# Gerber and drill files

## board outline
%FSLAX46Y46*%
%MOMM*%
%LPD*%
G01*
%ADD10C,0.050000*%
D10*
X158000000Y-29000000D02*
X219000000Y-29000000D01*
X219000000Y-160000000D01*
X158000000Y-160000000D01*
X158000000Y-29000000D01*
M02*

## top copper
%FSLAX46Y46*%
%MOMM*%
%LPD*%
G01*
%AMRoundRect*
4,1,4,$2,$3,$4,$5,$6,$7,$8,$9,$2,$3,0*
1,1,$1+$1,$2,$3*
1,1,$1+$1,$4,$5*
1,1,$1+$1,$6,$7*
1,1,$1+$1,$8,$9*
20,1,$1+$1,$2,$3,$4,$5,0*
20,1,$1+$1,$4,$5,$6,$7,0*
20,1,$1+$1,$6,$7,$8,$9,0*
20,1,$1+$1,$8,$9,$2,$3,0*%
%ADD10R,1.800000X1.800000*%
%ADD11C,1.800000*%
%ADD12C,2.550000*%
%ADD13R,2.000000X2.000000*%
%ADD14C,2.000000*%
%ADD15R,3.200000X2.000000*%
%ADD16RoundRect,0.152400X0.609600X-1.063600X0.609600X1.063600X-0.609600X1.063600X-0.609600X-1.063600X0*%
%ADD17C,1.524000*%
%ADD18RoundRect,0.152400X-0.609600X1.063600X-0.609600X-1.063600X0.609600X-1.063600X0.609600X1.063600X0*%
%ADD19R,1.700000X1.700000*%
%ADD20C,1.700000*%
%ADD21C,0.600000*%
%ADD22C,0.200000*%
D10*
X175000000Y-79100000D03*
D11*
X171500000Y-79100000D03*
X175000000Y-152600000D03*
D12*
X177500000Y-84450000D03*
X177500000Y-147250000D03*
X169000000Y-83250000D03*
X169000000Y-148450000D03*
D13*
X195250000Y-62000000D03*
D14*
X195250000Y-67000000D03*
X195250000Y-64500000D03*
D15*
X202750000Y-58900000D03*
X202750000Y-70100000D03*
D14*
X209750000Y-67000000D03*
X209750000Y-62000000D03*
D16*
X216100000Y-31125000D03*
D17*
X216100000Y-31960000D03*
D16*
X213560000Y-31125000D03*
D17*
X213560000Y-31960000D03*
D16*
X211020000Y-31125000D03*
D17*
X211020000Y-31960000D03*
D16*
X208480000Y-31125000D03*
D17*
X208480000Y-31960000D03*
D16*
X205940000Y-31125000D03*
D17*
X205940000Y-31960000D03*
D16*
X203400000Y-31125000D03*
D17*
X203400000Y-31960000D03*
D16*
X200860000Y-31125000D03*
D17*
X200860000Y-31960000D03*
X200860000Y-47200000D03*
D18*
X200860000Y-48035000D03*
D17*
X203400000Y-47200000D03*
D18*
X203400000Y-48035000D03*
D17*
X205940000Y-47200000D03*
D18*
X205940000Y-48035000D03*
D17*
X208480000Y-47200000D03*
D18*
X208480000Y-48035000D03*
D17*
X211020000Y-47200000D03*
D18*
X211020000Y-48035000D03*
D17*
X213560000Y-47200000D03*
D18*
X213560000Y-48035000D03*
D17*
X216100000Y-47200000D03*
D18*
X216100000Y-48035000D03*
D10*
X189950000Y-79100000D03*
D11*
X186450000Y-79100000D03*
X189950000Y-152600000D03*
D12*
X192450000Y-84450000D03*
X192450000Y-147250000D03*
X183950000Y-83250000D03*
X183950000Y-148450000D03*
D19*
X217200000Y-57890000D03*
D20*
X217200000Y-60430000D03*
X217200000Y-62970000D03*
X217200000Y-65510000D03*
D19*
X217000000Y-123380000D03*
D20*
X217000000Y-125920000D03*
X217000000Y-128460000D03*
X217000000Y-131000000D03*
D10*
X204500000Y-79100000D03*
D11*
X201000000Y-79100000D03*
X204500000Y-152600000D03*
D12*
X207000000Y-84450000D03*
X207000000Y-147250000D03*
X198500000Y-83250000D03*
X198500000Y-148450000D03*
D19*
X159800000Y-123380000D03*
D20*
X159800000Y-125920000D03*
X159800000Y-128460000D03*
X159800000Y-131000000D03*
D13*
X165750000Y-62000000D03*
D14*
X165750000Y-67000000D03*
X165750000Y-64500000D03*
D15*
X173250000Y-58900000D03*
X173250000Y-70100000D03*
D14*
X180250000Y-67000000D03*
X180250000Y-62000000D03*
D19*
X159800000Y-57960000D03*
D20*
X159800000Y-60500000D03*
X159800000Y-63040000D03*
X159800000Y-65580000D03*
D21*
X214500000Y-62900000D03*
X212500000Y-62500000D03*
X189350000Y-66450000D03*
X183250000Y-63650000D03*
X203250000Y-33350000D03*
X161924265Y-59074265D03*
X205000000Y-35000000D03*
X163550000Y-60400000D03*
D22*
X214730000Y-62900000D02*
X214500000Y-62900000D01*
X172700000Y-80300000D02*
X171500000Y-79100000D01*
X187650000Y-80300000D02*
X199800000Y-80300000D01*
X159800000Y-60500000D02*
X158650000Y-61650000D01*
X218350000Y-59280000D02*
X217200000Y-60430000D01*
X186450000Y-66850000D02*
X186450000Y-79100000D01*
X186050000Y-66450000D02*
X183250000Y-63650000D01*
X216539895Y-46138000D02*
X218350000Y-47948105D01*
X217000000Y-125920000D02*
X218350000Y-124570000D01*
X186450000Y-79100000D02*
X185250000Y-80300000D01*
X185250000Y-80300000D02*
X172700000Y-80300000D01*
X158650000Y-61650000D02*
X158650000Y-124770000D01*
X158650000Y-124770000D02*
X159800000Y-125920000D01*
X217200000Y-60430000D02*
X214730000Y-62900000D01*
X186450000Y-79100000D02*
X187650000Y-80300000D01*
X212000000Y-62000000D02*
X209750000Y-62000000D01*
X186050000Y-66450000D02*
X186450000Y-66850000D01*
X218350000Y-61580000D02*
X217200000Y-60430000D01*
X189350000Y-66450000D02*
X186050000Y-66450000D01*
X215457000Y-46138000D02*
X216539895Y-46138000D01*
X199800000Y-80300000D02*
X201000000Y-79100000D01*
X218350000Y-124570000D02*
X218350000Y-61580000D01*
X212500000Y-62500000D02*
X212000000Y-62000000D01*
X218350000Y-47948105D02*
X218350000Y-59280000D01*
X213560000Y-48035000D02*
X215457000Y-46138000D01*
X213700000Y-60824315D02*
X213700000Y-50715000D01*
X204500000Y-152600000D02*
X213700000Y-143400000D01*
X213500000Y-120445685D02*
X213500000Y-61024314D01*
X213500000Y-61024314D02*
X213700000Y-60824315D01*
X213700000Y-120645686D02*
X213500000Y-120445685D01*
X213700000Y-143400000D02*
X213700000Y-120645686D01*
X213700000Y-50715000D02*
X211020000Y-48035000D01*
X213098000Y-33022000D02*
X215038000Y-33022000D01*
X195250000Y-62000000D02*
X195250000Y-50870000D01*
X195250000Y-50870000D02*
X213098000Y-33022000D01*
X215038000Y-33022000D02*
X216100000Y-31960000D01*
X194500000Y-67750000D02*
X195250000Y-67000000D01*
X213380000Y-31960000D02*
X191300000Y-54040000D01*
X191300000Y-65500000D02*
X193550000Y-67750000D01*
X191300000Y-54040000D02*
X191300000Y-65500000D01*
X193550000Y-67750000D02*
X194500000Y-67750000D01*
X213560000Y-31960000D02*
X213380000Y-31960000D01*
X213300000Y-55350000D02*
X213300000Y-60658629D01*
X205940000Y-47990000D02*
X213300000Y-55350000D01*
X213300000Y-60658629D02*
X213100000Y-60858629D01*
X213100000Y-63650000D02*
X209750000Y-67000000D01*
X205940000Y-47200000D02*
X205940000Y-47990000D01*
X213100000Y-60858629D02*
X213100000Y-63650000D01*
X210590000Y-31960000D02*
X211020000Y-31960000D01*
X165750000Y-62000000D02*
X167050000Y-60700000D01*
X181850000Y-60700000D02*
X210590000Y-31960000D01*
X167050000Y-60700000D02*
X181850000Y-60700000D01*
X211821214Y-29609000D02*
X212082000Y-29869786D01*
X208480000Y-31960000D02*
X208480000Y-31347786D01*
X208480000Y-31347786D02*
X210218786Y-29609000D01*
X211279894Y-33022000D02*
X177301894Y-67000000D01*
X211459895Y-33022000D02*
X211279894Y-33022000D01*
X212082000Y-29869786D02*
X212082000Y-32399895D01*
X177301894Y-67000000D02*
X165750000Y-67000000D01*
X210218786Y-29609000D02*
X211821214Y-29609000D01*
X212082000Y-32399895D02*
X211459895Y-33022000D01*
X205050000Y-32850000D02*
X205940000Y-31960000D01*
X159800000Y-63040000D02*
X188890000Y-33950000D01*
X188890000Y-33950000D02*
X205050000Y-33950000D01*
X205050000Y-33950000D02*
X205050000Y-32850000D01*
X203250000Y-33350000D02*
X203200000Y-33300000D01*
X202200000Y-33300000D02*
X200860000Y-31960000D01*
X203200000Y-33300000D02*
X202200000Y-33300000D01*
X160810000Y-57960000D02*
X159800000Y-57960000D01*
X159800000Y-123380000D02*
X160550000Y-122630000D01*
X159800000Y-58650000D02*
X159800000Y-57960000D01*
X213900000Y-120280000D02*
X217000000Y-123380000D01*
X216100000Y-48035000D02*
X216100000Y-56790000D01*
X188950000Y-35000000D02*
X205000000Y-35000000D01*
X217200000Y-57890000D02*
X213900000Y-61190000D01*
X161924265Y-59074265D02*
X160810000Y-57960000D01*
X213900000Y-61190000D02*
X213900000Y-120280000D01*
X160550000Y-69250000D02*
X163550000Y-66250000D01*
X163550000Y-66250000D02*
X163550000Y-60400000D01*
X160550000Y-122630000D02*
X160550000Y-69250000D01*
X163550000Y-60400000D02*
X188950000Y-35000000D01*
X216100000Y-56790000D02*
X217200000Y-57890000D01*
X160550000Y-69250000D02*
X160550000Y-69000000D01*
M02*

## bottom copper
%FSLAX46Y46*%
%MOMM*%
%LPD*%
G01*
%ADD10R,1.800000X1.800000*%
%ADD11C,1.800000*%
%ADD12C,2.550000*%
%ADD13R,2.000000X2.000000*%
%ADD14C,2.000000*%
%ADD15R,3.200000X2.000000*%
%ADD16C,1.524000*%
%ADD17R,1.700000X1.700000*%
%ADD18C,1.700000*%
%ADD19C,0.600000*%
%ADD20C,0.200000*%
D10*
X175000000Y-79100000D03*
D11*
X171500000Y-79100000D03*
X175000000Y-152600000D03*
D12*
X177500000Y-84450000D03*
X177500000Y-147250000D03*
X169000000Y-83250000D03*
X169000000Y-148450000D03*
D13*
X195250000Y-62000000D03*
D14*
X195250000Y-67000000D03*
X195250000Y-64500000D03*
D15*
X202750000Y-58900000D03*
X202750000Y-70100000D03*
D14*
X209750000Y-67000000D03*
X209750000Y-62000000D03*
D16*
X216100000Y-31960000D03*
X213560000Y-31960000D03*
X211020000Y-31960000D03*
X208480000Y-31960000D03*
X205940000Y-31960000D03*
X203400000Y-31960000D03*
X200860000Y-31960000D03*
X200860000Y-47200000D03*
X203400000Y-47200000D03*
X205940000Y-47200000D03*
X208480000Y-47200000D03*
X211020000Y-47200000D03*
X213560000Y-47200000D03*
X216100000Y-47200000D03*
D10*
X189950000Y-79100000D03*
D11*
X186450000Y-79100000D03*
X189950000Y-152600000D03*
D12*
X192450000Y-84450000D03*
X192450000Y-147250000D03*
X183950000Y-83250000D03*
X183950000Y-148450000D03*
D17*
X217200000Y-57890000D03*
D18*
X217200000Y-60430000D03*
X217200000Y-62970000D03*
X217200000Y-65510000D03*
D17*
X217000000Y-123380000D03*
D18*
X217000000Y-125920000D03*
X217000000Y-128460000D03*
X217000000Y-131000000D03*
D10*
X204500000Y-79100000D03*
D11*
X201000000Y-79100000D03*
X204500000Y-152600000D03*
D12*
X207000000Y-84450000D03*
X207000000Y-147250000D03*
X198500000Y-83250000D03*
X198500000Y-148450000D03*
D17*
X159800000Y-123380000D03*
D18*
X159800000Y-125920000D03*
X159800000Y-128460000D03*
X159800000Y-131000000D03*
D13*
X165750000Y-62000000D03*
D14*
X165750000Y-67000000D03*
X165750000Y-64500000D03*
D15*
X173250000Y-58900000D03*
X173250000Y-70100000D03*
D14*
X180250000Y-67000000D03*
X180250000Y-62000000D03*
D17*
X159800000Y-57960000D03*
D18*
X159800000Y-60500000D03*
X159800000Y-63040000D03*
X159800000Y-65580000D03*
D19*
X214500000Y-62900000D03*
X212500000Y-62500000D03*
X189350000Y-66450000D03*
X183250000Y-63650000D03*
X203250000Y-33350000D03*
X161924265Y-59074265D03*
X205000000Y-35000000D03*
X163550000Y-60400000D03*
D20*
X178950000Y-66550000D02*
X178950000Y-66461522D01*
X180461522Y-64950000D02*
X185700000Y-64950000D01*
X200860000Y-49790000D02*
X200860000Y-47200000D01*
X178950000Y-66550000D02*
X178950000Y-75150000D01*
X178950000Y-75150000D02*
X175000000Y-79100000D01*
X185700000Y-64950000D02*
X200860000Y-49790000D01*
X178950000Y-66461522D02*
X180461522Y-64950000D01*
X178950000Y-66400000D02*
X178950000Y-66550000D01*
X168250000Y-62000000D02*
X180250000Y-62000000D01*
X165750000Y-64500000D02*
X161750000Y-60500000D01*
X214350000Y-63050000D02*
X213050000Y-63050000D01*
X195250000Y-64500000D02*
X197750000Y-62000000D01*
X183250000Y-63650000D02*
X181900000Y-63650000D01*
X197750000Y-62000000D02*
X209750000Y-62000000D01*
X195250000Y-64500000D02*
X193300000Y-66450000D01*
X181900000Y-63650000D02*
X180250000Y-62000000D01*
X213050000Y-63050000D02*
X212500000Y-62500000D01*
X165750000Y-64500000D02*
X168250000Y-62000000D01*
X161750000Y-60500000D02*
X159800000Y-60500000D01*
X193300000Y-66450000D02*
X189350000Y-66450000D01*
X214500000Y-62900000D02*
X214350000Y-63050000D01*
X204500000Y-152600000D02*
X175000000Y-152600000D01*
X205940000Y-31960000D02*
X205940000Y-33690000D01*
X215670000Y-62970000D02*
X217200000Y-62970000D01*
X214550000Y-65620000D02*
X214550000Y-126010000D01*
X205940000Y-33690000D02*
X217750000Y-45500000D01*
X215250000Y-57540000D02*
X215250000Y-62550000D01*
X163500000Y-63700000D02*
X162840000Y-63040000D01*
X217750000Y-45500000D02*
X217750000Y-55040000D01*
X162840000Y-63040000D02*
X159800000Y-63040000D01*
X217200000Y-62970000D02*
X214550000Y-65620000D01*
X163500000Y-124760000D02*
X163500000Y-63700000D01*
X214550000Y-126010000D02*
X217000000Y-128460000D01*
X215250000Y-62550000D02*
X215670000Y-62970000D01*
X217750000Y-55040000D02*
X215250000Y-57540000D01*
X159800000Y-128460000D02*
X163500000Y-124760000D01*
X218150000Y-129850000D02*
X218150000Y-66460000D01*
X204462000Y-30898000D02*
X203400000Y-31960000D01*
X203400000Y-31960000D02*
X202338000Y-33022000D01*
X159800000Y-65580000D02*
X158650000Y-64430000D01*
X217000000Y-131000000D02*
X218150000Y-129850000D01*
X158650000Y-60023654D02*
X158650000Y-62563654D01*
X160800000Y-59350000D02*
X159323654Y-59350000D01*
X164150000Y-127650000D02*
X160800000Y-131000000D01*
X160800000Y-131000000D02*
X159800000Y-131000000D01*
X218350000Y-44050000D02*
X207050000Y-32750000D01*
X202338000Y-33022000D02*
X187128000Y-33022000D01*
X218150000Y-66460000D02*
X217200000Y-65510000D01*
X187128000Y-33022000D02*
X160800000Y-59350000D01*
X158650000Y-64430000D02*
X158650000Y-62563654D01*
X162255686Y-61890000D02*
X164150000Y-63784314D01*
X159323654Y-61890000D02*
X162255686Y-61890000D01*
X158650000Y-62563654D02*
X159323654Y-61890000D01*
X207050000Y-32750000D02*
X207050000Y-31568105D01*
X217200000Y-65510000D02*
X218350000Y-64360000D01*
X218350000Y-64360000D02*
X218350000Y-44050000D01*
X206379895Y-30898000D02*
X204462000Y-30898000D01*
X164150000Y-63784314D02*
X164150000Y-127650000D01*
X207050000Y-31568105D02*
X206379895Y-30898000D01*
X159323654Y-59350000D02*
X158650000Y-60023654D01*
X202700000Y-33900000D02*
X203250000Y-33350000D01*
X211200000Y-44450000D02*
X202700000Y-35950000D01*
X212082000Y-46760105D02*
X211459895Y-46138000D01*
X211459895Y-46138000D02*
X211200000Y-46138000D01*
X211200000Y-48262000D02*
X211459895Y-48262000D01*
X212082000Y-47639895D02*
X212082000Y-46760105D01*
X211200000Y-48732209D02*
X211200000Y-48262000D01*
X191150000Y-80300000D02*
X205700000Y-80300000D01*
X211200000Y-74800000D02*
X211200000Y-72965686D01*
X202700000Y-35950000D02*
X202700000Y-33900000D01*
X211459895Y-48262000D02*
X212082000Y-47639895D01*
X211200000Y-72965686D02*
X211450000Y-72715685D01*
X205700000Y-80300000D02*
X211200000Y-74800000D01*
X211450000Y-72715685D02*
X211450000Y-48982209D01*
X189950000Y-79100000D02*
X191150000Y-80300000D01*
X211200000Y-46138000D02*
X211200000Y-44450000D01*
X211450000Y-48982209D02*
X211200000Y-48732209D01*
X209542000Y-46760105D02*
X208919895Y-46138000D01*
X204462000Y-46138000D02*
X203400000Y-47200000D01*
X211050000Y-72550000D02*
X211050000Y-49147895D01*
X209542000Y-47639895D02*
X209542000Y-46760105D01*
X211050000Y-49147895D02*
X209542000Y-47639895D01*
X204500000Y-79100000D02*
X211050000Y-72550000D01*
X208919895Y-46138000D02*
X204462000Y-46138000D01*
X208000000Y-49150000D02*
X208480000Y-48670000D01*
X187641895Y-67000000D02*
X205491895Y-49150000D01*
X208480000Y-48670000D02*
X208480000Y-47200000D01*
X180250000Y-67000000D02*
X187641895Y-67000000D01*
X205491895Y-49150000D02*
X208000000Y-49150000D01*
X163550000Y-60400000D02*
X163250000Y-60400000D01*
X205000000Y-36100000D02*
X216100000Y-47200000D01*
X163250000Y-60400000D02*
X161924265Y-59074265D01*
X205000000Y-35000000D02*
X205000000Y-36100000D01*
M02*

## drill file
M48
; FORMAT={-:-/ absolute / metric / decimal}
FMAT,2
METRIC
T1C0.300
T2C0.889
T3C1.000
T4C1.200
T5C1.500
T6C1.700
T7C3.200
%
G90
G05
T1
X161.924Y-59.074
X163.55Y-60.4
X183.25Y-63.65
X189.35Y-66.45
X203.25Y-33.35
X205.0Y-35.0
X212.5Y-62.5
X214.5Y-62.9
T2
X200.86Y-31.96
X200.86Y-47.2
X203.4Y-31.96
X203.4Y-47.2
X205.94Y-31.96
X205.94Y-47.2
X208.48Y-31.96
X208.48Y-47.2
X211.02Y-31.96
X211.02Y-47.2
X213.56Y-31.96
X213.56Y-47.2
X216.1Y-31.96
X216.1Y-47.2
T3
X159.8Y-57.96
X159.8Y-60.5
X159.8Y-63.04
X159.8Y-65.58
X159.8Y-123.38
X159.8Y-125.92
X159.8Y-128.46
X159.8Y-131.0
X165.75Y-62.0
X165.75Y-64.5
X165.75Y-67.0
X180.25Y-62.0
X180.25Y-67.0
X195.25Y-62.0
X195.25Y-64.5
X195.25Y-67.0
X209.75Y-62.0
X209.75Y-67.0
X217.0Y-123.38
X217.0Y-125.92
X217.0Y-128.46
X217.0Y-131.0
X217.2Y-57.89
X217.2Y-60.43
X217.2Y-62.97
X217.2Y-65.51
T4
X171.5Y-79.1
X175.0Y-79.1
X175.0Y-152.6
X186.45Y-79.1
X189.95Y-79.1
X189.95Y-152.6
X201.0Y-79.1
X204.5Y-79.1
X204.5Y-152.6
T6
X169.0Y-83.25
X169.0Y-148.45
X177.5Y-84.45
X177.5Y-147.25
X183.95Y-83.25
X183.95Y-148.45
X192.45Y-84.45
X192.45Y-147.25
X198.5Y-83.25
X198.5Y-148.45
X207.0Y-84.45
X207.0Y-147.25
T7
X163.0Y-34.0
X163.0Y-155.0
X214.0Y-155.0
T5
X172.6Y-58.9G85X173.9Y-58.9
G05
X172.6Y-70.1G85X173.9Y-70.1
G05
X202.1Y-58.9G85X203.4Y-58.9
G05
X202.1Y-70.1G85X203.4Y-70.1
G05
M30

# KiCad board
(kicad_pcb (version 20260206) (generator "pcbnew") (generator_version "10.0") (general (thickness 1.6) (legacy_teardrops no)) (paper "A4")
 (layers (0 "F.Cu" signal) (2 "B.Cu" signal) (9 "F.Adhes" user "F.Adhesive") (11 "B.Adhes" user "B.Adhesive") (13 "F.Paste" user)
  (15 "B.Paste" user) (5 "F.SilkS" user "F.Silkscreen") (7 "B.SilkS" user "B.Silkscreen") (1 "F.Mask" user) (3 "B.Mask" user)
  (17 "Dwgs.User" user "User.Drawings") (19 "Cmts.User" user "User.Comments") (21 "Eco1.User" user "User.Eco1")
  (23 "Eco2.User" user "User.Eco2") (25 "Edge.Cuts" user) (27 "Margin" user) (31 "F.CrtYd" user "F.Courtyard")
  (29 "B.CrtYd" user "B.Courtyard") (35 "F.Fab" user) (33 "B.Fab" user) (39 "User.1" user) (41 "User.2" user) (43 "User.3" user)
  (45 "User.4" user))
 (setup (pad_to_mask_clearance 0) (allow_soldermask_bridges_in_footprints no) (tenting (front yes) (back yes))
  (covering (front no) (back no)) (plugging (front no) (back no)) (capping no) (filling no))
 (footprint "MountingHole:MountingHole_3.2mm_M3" (layer "F.Cu") (at 163 34)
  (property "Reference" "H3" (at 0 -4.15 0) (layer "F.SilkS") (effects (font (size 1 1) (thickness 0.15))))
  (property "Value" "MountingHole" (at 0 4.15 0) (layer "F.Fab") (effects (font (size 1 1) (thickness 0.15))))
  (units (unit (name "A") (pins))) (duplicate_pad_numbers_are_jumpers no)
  (pad "" np_thru_hole circle (at 0 0) (size 3.2 3.2) (drill 3.2) (layers "*.Cu" "*.Mask")))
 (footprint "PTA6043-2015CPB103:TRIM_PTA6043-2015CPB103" (layer "F.Cu") (at 173.25 115.85 -90)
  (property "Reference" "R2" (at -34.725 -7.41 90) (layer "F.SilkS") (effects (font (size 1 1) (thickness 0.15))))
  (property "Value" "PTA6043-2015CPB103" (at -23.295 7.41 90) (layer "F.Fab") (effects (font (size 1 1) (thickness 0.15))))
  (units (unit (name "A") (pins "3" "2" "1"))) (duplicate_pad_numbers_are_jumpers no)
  (pad "1" thru_hole rect (at -36.75 -1.75 270) (size 1.8 1.8) (drill 1.2) (layers "*.Cu" "*.Mask") (remove_unused_layers no) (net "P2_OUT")
   (solder_mask_margin 0.102))
  (pad "2" thru_hole circle (at -36.75 1.75 270) (size 1.8 1.8) (drill 1.2) (layers "*.Cu" "*.Mask") (remove_unused_layers no) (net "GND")
   (solder_mask_margin 0.102))
  (pad "3" thru_hole circle (at 36.75 -1.75 270) (size 1.8 1.8) (drill 1.2) (layers "*.Cu" "*.Mask") (remove_unused_layers no) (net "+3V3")
   (solder_mask_margin 0.102))
  (pad "SH1" thru_hole circle (at -31.4 -4.25 270) (size 2.55 2.55) (drill 1.7) (layers "*.Cu" "*.Mask") (remove_unused_layers no)
   (solder_mask_margin 0.102))
  (pad "SH2" thru_hole circle (at 31.4 -4.25 270) (size 2.55 2.55) (drill 1.7) (layers "*.Cu" "*.Mask") (remove_unused_layers no)
   (solder_mask_margin 0.102))
  (pad "SH3" thru_hole circle (at -32.6 4.25 270) (size 2.55 2.55) (drill 1.7) (layers "*.Cu" "*.Mask") (remove_unused_layers no)
   (solder_mask_margin 0.102))
  (pad "SH4" thru_hole circle (at 32.6 4.25 270) (size 2.55 2.55) (drill 1.7) (layers "*.Cu" "*.Mask") (remove_unused_layers no)
   (solder_mask_margin 0.102)))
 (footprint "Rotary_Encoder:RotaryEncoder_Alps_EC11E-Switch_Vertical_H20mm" (layer "F.Cu") (at 195.25 62)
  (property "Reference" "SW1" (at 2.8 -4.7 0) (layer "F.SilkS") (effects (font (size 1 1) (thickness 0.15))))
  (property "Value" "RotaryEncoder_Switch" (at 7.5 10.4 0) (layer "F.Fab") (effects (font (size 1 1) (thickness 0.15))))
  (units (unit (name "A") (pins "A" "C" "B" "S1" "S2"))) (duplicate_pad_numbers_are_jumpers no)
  (pad "A" thru_hole rect (at 0 0) (size 2 2) (drill 1) (layers "*.Cu" "*.Mask") (remove_unused_layers no) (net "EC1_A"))
  (pad "B" thru_hole circle (at 0 5) (size 2 2) (drill 1) (layers "*.Cu" "*.Mask") (remove_unused_layers no) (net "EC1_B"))
  (pad "C" thru_hole circle (at 0 2.5) (size 2 2) (drill 1) (layers "*.Cu" "*.Mask") (remove_unused_layers no) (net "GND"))
  (pad "MP" thru_hole rect (at 7.5 -3.1) (size 3.2 2) (drill oval 2.8 1.5) (layers "*.Cu" "*.Mask") (remove_unused_layers no))
  (pad "MP" thru_hole rect (at 7.5 8.1) (size 3.2 2) (drill oval 2.8 1.5) (layers "*.Cu" "*.Mask") (remove_unused_layers no))
  (pad "S1" thru_hole circle (at 14.5 5) (size 2 2) (drill 1) (layers "*.Cu" "*.Mask") (remove_unused_layers no) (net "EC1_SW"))
  (pad "S2" thru_hole circle (at 14.5 0) (size 2 2) (drill 1) (layers "*.Cu" "*.Mask") (remove_unused_layers no) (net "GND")))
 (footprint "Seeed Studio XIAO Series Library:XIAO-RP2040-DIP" (layer "F.Cu") (at 208.48 39.58)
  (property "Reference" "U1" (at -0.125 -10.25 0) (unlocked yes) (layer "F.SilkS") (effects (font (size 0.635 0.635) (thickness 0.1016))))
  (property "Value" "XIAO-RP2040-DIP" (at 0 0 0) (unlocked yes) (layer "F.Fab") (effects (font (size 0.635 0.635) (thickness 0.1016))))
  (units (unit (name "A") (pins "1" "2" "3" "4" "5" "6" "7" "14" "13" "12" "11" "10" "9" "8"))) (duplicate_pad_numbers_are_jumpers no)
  (pad "1" smd roundrect (at 7.62 -8.455 90) (size 2.432 1.524) (layers "F.Cu" "F.Mask") (roundrect_rratio 0.1) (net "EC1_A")
   (thermal_bridge_angle 45))
  (pad "1" thru_hole circle (at 7.62 -7.62 90) (size 1.524 1.524) (drill 0.889) (layers "*.Cu" "*.Mask") (remove_unused_layers no)
   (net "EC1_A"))
  (pad "2" smd roundrect (at 5.08 -8.455 90) (size 2.432 1.524) (layers "F.Cu" "F.Mask") (roundrect_rratio 0.1) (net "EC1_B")
   (thermal_bridge_angle 45))
  (pad "2" thru_hole circle (at 5.08 -7.62 90) (size 1.524 1.524) (drill 0.889) (layers "*.Cu" "*.Mask") (remove_unused_layers no)
   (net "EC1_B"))
  (pad "3" smd roundrect (at 2.54 -8.455 90) (size 2.432 1.524) (layers "F.Cu" "F.Mask") (roundrect_rratio 0.1) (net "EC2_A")
   (thermal_bridge_angle 45))
  (pad "3" thru_hole circle (at 2.54 -7.62 90) (size 1.524 1.524) (drill 0.889) (layers "*.Cu" "*.Mask") (remove_unused_layers no)
   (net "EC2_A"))
  (pad "4" smd roundrect (at 0 -8.455 90) (size 2.432 1.524) (layers "F.Cu" "F.Mask") (roundrect_rratio 0.1) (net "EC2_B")
   (thermal_bridge_angle 45))
  (pad "4" thru_hole circle (at 0 -7.62 90) (size 1.524 1.524) (drill 0.889) (layers "*.Cu" "*.Mask") (remove_unused_layers no)
   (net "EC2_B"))
  (pad "5" smd roundrect (at -2.54 -8.455 90) (size 2.432 1.524) (layers "F.Cu" "F.Mask") (roundrect_rratio 0.1) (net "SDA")
   (thermal_bridge_angle 45))
  (pad "5" thru_hole circle (at -2.54 -7.62 90) (size 1.524 1.524) (drill 0.889) (layers "*.Cu" "*.Mask") (remove_unused_layers no)
   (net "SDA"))
  (pad "6" smd roundrect (at -5.08 -8.455 90) (size 2.432 1.524) (layers "F.Cu" "F.Mask") (roundrect_rratio 0.1) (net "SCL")
   (thermal_bridge_angle 45))
  (pad "6" thru_hole circle (at -5.08 -7.62 90) (size 1.524 1.524) (drill 0.889) (layers "*.Cu" "*.Mask") (remove_unused_layers no)
   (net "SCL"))
  (pad "7" smd roundrect (at -7.62 -8.455 90) (size 2.432 1.524) (layers "F.Cu" "F.Mask") (roundrect_rratio 0.1) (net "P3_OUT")
   (thermal_bridge_angle 45))
  (pad "7" thru_hole circle (at -7.62 -7.62 90) (size 1.524 1.524) (drill 0.889) (layers "*.Cu" "*.Mask") (remove_unused_layers no)
   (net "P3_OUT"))
  (pad "8" thru_hole circle (at -7.62 7.62 270) (size 1.524 1.524) (drill 0.889) (layers "*.Cu" "*.Mask") (remove_unused_layers no)
   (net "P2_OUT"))
  (pad "8" smd roundrect (at -7.62 8.455 270) (size 2.432 1.524) (layers "F.Cu" "F.Mask") (roundrect_rratio 0.1) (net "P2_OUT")
   (thermal_bridge_angle 45))
  (pad "9" thru_hole circle (at -5.08 7.62 270) (size 1.524 1.524) (drill 0.889) (layers "*.Cu" "*.Mask") (remove_unused_layers no)
   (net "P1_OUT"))
  (pad "9" smd roundrect (at -5.08 8.455 270) (size 2.432 1.524) (layers "F.Cu" "F.Mask") (roundrect_rratio 0.1) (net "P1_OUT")
   (thermal_bridge_angle 45))
  (pad "10" thru_hole circle (at -2.54 7.62 270) (size 1.524 1.524) (drill 0.889) (layers "*.Cu" "*.Mask") (remove_unused_layers no)
   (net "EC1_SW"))
  (pad "10" smd roundrect (at -2.54 8.455 270) (size 2.432 1.524) (layers "F.Cu" "F.Mask") (roundrect_rratio 0.1) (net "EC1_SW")
   (thermal_bridge_angle 45))
  (pad "11" thru_hole circle (at 0 7.62 270) (size 1.524 1.524) (drill 0.889) (layers "*.Cu" "*.Mask") (remove_unused_layers no)
   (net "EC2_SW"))
  (pad "11" smd roundrect (at 0 8.455 270) (size 2.432 1.524) (layers "F.Cu" "F.Mask") (roundrect_rratio 0.1) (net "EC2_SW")
   (thermal_bridge_angle 45))
  (pad "12" thru_hole circle (at 2.54 7.62 270) (size 1.524 1.524) (drill 0.889) (layers "*.Cu" "*.Mask") (remove_unused_layers no)
   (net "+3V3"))
  (pad "12" smd roundrect (at 2.54 8.455 270) (size 2.432 1.524) (layers "F.Cu" "F.Mask") (roundrect_rratio 0.1) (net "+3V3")
   (thermal_bridge_angle 45))
  (pad "13" thru_hole circle (at 5.08 7.62 270) (size 1.524 1.524) (drill 0.889) (layers "*.Cu" "*.Mask") (remove_unused_layers no)
   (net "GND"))
  (pad "13" smd roundrect (at 5.08 8.455 270) (size 2.432 1.524) (layers "F.Cu" "F.Mask") (roundrect_rratio 0.1) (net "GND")
   (thermal_bridge_angle 45))
  (pad "14" thru_hole circle (at 7.62 7.62 270) (size 1.524 1.524) (drill 0.889) (layers "*.Cu" "*.Mask") (remove_unused_layers no)
   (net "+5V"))
  (pad "14" smd roundrect (at 7.62 8.455 270) (size 2.432 1.524) (layers "F.Cu" "F.Mask") (roundrect_rratio 0.1) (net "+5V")
   (thermal_bridge_angle 45)))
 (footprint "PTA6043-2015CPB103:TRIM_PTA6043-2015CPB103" (layer "F.Cu") (at 188.2 115.85 -90)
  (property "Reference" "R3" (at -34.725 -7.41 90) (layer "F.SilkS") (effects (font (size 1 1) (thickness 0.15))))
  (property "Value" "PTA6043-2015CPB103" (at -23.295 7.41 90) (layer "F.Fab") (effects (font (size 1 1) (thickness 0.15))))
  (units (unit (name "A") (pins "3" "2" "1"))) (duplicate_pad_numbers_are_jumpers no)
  (pad "1" thru_hole rect (at -36.75 -1.75 270) (size 1.8 1.8) (drill 1.2) (layers "*.Cu" "*.Mask") (remove_unused_layers no) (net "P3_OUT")
   (solder_mask_margin 0.102))
  (pad "2" thru_hole circle (at -36.75 1.75 270) (size 1.8 1.8) (drill 1.2) (layers "*.Cu" "*.Mask") (remove_unused_layers no) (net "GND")
   (solder_mask_margin 0.102))
  (pad "3" thru_hole circle (at 36.75 -1.75 270) (size 1.8 1.8) (drill 1.2) (layers "*.Cu" "*.Mask") (remove_unused_layers no) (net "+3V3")
   (solder_mask_margin 0.102))
  (pad "SH1" thru_hole circle (at -31.4 -4.25 270) (size 2.55 2.55) (drill 1.7) (layers "*.Cu" "*.Mask") (remove_unused_layers no)
   (solder_mask_margin 0.102))
  (pad "SH2" thru_hole circle (at 31.4 -4.25 270) (size 2.55 2.55) (drill 1.7) (layers "*.Cu" "*.Mask") (remove_unused_layers no)
   (solder_mask_margin 0.102))
  (pad "SH3" thru_hole circle (at -32.6 4.25 270) (size 2.55 2.55) (drill 1.7) (layers "*.Cu" "*.Mask") (remove_unused_layers no)
   (solder_mask_margin 0.102))
  (pad "SH4" thru_hole circle (at 32.6 4.25 270) (size 2.55 2.55) (drill 1.7) (layers "*.Cu" "*.Mask") (remove_unused_layers no)
   (solder_mask_margin 0.102)))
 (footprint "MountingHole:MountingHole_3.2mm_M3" (layer "F.Cu") (at 163 155)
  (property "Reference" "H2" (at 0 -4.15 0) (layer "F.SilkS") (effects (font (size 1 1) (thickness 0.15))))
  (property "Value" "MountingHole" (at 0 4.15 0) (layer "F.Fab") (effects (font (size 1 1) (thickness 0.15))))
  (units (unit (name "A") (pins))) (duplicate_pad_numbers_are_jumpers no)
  (pad "" np_thru_hole circle (at 0 0) (size 3.2 3.2) (drill 3.2) (layers "*.Cu" "*.Mask")))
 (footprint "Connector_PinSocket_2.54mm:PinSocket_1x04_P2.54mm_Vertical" (layer "F.Cu") (at 217.2 57.89)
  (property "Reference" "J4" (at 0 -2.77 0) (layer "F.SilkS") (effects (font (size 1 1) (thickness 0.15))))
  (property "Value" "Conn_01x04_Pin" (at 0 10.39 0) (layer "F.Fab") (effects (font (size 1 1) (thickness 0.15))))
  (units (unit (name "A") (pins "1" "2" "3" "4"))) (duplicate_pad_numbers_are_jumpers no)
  (pad "1" thru_hole rect (at 0 0) (size 1.7 1.7) (drill 1) (layers "*.Cu" "*.Mask") (remove_unused_layers no) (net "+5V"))
  (pad "2" thru_hole circle (at 0 2.54) (size 1.7 1.7) (drill 1) (layers "*.Cu" "*.Mask") (remove_unused_layers no) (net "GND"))
  (pad "3" thru_hole circle (at 0 5.08) (size 1.7 1.7) (drill 1) (layers "*.Cu" "*.Mask") (remove_unused_layers no) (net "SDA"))
  (pad "4" thru_hole circle (at 0 7.62) (size 1.7 1.7) (drill 1) (layers "*.Cu" "*.Mask") (remove_unused_layers no) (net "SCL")))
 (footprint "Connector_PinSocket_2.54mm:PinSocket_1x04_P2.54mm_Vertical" (layer "F.Cu") (at 217 123.38)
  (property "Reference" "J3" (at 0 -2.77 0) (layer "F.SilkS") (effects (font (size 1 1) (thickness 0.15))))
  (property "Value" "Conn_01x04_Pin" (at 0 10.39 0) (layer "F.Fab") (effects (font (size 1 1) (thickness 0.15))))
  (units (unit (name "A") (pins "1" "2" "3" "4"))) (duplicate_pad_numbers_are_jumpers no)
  (pad "1" thru_hole rect (at 0 0) (size 1.7 1.7) (drill 1) (layers "*.Cu" "*.Mask") (remove_unused_layers no) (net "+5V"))
  (pad "2" thru_hole circle (at 0 2.54) (size 1.7 1.7) (drill 1) (layers "*.Cu" "*.Mask") (remove_unused_layers no) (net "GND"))
  (pad "3" thru_hole circle (at 0 5.08) (size 1.7 1.7) (drill 1) (layers "*.Cu" "*.Mask") (remove_unused_layers no) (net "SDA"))
  (pad "4" thru_hole circle (at 0 7.62) (size 1.7 1.7) (drill 1) (layers "*.Cu" "*.Mask") (remove_unused_layers no) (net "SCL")))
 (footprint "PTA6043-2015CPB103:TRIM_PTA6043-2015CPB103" (layer "F.Cu") (at 202.75 115.85 -90)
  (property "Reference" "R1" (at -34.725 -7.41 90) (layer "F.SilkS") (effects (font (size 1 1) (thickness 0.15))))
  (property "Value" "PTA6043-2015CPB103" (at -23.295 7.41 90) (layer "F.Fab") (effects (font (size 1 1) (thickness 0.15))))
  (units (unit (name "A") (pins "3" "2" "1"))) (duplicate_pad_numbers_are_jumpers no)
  (pad "1" thru_hole rect (at -36.75 -1.75 270) (size 1.8 1.8) (drill 1.2) (layers "*.Cu" "*.Mask") (remove_unused_layers no) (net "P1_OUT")
   (solder_mask_margin 0.102))
  (pad "2" thru_hole circle (at -36.75 1.75 270) (size 1.8 1.8) (drill 1.2) (layers "*.Cu" "*.Mask") (remove_unused_layers no) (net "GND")
   (solder_mask_margin 0.102))
  (pad "3" thru_hole circle (at 36.75 -1.75 270) (size 1.8 1.8) (drill 1.2) (layers "*.Cu" "*.Mask") (remove_unused_layers no) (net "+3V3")
   (solder_mask_margin 0.102))
  (pad "SH1" thru_hole circle (at -31.4 -4.25 270) (size 2.55 2.55) (drill 1.7) (layers "*.Cu" "*.Mask") (remove_unused_layers no)
   (solder_mask_margin 0.102))
  (pad "SH2" thru_hole circle (at 31.4 -4.25 270) (size 2.55 2.55) (drill 1.7) (layers "*.Cu" "*.Mask") (remove_unused_layers no)
   (solder_mask_margin 0.102))
  (pad "SH3" thru_hole circle (at -32.6 4.25 270) (size 2.55 2.55) (drill 1.7) (layers "*.Cu" "*.Mask") (remove_unused_layers no)
   (solder_mask_margin 0.102))
  (pad "SH4" thru_hole circle (at 32.6 4.25 270) (size 2.55 2.55) (drill 1.7) (layers "*.Cu" "*.Mask") (remove_unused_layers no)
   (solder_mask_margin 0.102)))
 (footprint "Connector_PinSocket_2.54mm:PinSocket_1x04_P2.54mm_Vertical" (layer "F.Cu") (at 159.8 123.38)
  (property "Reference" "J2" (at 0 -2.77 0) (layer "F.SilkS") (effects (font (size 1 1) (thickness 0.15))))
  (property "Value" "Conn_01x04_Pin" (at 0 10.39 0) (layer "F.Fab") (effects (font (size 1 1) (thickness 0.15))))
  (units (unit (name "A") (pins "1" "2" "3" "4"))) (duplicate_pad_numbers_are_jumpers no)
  (pad "1" thru_hole rect (at 0 0) (size 1.7 1.7) (drill 1) (layers "*.Cu" "*.Mask") (remove_unused_layers no) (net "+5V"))
  (pad "2" thru_hole circle (at 0 2.54) (size 1.7 1.7) (drill 1) (layers "*.Cu" "*.Mask") (remove_unused_layers no) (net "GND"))
  (pad "3" thru_hole circle (at 0 5.08) (size 1.7 1.7) (drill 1) (layers "*.Cu" "*.Mask") (remove_unused_layers no) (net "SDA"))
  (pad "4" thru_hole circle (at 0 7.62) (size 1.7 1.7) (drill 1) (layers "*.Cu" "*.Mask") (remove_unused_layers no) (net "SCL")))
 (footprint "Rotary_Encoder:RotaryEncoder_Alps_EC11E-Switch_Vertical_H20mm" (layer "F.Cu") (at 165.75 62)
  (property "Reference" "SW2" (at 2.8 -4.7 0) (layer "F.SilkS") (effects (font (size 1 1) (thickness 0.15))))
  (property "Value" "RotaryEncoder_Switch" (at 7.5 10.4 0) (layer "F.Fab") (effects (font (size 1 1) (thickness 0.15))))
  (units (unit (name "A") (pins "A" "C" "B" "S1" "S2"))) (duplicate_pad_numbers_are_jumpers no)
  (pad "A" thru_hole rect (at 0 0) (size 2 2) (drill 1) (layers "*.Cu" "*.Mask") (remove_unused_layers no) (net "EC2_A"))
  (pad "B" thru_hole circle (at 0 5) (size 2 2) (drill 1) (layers "*.Cu" "*.Mask") (remove_unused_layers no) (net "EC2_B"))
  (pad "C" thru_hole circle (at 0 2.5) (size 2 2) (drill 1) (layers "*.Cu" "*.Mask") (remove_unused_layers no) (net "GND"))
  (pad "MP" thru_hole rect (at 7.5 -3.1) (size 3.2 2) (drill oval 2.8 1.5) (layers "*.Cu" "*.Mask") (remove_unused_layers no))
  (pad "MP" thru_hole rect (at 7.5 8.1) (size 3.2 2) (drill oval 2.8 1.5) (layers "*.Cu" "*.Mask") (remove_unused_layers no))
  (pad "S1" thru_hole circle (at 14.5 5) (size 2 2) (drill 1) (layers "*.Cu" "*.Mask") (remove_unused_layers no) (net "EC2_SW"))
  (pad "S2" thru_hole circle (at 14.5 0) (size 2 2) (drill 1) (layers "*.Cu" "*.Mask") (remove_unused_layers no) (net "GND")))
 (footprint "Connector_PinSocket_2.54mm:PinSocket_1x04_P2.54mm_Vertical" (layer "F.Cu") (at 159.8 57.96)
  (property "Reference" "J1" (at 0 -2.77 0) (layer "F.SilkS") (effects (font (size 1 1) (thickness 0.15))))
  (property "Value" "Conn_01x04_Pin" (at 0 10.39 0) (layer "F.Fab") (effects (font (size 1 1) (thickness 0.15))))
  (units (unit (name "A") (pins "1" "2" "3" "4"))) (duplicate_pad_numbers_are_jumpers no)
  (pad "1" thru_hole rect (at 0 0) (size 1.7 1.7) (drill 1) (layers "*.Cu" "*.Mask") (remove_unused_layers no) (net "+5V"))
  (pad "2" thru_hole circle (at 0 2.54) (size 1.7 1.7) (drill 1) (layers "*.Cu" "*.Mask") (remove_unused_layers no) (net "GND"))
  (pad "3" thru_hole circle (at 0 5.08) (size 1.7 1.7) (drill 1) (layers "*.Cu" "*.Mask") (remove_unused_layers no) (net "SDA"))
  (pad "4" thru_hole circle (at 0 7.62) (size 1.7 1.7) (drill 1) (layers "*.Cu" "*.Mask") (remove_unused_layers no) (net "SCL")))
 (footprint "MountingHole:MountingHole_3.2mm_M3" (layer "F.Cu") (at 214 155)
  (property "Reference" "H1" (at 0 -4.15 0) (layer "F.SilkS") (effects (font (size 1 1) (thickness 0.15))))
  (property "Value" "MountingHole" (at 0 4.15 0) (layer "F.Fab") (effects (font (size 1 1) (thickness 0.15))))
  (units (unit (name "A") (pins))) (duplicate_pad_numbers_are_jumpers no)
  (pad "" np_thru_hole circle (at 0 0) (size 3.2 3.2) (drill 3.2) (layers "*.Cu" "*.Mask")))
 (gr_rect (start 158 29) (end 219 160) (stroke (width 0.05) (type default)) (fill no) (layer "Edge.Cuts"))
 (segment (start 178.95 66.55) (end 178.95 66.461522) (width 0.2) (layer "B.Cu") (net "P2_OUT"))
 (segment (start 180.461522 64.95) (end 185.7 64.95) (width 0.2) (layer "B.Cu") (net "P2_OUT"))
 (segment (start 200.86 49.79) (end 200.86 47.2) (width 0.2) (layer "B.Cu") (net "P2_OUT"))
 (segment (start 178.95 66.55) (end 178.95 75.15) (width 0.2) (layer "B.Cu") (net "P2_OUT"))
 (segment (start 178.95 75.15) (end 175 79.1) (width 0.2) (layer "B.Cu") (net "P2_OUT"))
 (segment (start 185.7 64.95) (end 200.86 49.79) (width 0.2) (layer "B.Cu") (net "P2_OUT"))
 (segment (start 178.95 66.461522) (end 180.461522 64.95) (width 0.2) (layer "B.Cu") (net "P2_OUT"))
 (segment (start 178.95 66.4) (end 178.95 66.55) (width 0.2) (layer "B.Cu") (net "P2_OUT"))
 (segment (start 214.73 62.9) (end 214.5 62.9) (width 0.2) (layer "F.Cu") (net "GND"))
 (segment (start 172.7 80.3) (end 171.5 79.1) (width 0.2) (layer "F.Cu") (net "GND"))
 (segment (start 187.65 80.3) (end 199.8 80.3) (width 0.2) (layer "F.Cu") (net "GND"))
 (segment (start 159.8 60.5) (end 158.65 61.65) (width 0.2) (layer "F.Cu") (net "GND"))
 (segment (start 218.35 59.28) (end 217.2 60.43) (width 0.2) (layer "F.Cu") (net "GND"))
 (segment (start 186.45 66.85) (end 186.45 79.1) (width 0.2) (layer "F.Cu") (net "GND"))
 (segment (start 186.05 66.45) (end 183.25 63.65) (width 0.2) (layer "F.Cu") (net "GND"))
 (segment (start 216.539895 46.138) (end 218.35 47.948105) (width 0.2) (layer "F.Cu") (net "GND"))
 (segment (start 217 125.92) (end 218.35 124.57) (width 0.2) (layer "F.Cu") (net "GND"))
 (segment (start 186.45 79.1) (end 185.25 80.3) (width 0.2) (layer "F.Cu") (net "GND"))
 (segment (start 185.25 80.3) (end 172.7 80.3) (width 0.2) (layer "F.Cu") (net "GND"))
 (segment (start 158.65 61.65) (end 158.65 124.77) (width 0.2) (layer "F.Cu") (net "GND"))
 (segment (start 158.65 124.77) (end 159.8 125.92) (width 0.2) (layer "F.Cu") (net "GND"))
 (segment (start 217.2 60.43) (end 214.73 62.9) (width 0.2) (layer "F.Cu") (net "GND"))
 (segment (start 186.45 79.1) (end 187.65 80.3) (width 0.2) (layer "F.Cu") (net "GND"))
 (segment (start 212 62) (end 209.75 62) (width 0.2) (layer "F.Cu") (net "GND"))
 (segment (start 186.05 66.45) (end 186.45 66.85) (width 0.2) (layer "F.Cu") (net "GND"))
 (segment (start 218.35 61.58) (end 217.2 60.43) (width 0.2) (layer "F.Cu") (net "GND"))
 (segment (start 189.35 66.45) (end 186.05 66.45) (width 0.2) (layer "F.Cu") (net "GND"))
 (segment (start 215.457 46.138) (end 216.539895 46.138) (width 0.2) (layer "F.Cu") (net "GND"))
 (segment (start 199.8 80.3) (end 201 79.1) (width 0.2) (layer "F.Cu") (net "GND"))
 (segment (start 218.35 124.57) (end 218.35 61.58) (width 0.2) (layer "F.Cu") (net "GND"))
 (segment (start 212.5 62.5) (end 212 62) (width 0.2) (layer "F.Cu") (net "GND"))
 (segment (start 218.35 47.948105) (end 218.35 59.28) (width 0.2) (layer "F.Cu") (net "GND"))
 (segment (start 213.56 48.035) (end 215.457 46.138) (width 0.2) (layer "F.Cu") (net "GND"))
 (via (at 214.5 62.9) (size 0.6) (drill 0.3) (layers "F.Cu" "B.Cu") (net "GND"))
 (via (at 212.5 62.5) (size 0.6) (drill 0.3) (layers "F.Cu" "B.Cu") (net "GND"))
 (via (at 189.35 66.45) (size 0.6) (drill 0.3) (layers "F.Cu" "B.Cu") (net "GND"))
 (via (at 183.25 63.65) (size 0.6) (drill 0.3) (layers "F.Cu" "B.Cu") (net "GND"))
 (segment (start 168.25 62) (end 180.25 62) (width 0.2) (layer "B.Cu") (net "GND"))
 (segment (start 165.75 64.5) (end 161.75 60.5) (width 0.2) (layer "B.Cu") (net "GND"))
 (segment (start 214.35 63.05) (end 213.05 63.05) (width 0.2) (layer "B.Cu") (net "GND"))
 (segment (start 195.25 64.5) (end 197.75 62) (width 0.2) (layer "B.Cu") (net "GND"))
 (segment (start 183.25 63.65) (end 181.9 63.65) (width 0.2) (layer "B.Cu") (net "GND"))
 (segment (start 197.75 62) (end 209.75 62) (width 0.2) (layer "B.Cu") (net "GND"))
 (segment (start 195.25 64.5) (end 193.3 66.45) (width 0.2) (layer "B.Cu") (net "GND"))
 (segment (start 181.9 63.65) (end 180.25 62) (width 0.2) (layer "B.Cu") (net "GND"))
 (segment (start 213.05 63.05) (end 212.5 62.5) (width 0.2) (layer "B.Cu") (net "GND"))
 (segment (start 165.75 64.5) (end 168.25 62) (width 0.2) (layer "B.Cu") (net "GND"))
 (segment (start 161.75 60.5) (end 159.8 60.5) (width 0.2) (layer "B.Cu") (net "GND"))
 (segment (start 193.3 66.45) (end 189.35 66.45) (width 0.2) (layer "B.Cu") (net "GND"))
 (segment (start 214.5 62.9) (end 214.35 63.05) (width 0.2) (layer "B.Cu") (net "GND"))
 (segment (start 213.7 60.824315) (end 213.7 50.715) (width 0.2) (layer "F.Cu") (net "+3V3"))
 (segment (start 204.5 152.6) (end 213.7 143.4) (width 0.2) (layer "F.Cu") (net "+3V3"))
 (segment (start 213.5 120.445685) (end 213.5 61.024314) (width 0.2) (layer "F.Cu") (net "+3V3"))
 (segment (start 213.5 61.024314) (end 213.7 60.824315) (width 0.2) (layer "F.Cu") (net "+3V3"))
 (segment (start 213.7 120.645686) (end 213.5 120.445685) (width 0.2) (layer "F.Cu") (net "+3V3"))
 (segment (start 213.7 143.4) (end 213.7 120.645686) (width 0.2) (layer "F.Cu") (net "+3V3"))
 (segment (start 213.7 50.715) (end 211.02 48.035) (width 0.2) (layer "F.Cu") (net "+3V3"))
 (segment (start 204.5 152.6) (end 175 152.6) (width 0.2) (layer "B.Cu") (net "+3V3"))
 (segment (start 213.098 33.022) (end 215.038 33.022) (width 0.2) (layer "F.Cu") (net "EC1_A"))
 (segment (start 195.25 62) (end 195.25 50.87) (width 0.2) (layer "F.Cu") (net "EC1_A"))
 (segment (start 195.25 50.87) (end 213.098 33.022) (width 0.2) (layer "F.Cu") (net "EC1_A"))
 (segment (start 215.038 33.022) (end 216.1 31.96) (width 0.2) (layer "F.Cu") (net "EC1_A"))
 (segment (start 194.5 67.75) (end 195.25 67) (width 0.2) (layer "F.Cu") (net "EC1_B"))
 (segment (start 213.38 31.96) (end 191.3 54.04) (width 0.2) (layer "F.Cu") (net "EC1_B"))
 (segment (start 191.3 65.5) (end 193.55 67.75) (width 0.2) (layer "F.Cu") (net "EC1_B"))
 (segment (start 191.3 54.04) (end 191.3 65.5) (width 0.2) (layer "F.Cu") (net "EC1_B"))
 (segment (start 193.55 67.75) (end 194.5 67.75) (width 0.2) (layer "F.Cu") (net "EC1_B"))
 (segment (start 213.56 31.96) (end 213.38 31.96) (width 0.2) (layer "F.Cu") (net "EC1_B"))
 (segment (start 213.3 55.35) (end 213.3 60.658629) (width 0.2) (layer "F.Cu") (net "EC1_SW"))
 (segment (start 205.94 47.99) (end 213.3 55.35) (width 0.2) (layer "F.Cu") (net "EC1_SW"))
 (segment (start 213.3 60.658629) (end 213.1 60.858629) (width 0.2) (layer "F.Cu") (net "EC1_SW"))
 (segment (start 213.1 63.65) (end 209.75 67) (width 0.2) (layer "F.Cu") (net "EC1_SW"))
 (segment (start 205.94 47.2) (end 205.94 47.99) (width 0.2) (layer "F.Cu") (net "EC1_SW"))
 (segment (start 213.1 60.858629) (end 213.1 63.65) (width 0.2) (layer "F.Cu") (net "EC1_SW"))
 (segment (start 210.59 31.96) (end 211.02 31.96) (width 0.2) (layer "F.Cu") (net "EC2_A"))
 (segment (start 165.75 62) (end 167.05 60.7) (width 0.2) (layer "F.Cu") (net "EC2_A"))
 (segment (start 181.85 60.7) (end 210.59 31.96) (width 0.2) (layer "F.Cu") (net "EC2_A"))
 (segment (start 167.05 60.7) (end 181.85 60.7) (width 0.2) (layer "F.Cu") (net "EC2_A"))
 (segment (start 211.821214 29.609) (end 212.082 29.869786) (width 0.2) (layer "F.Cu") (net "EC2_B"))
 (segment (start 208.48 31.96) (end 208.48 31.347786) (width 0.2) (layer "F.Cu") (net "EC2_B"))
 (segment (start 208.48 31.347786) (end 210.218786 29.609) (width 0.2) (layer "F.Cu") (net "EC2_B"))
 (segment (start 211.279894 33.022) (end 177.301894 67) (width 0.2) (layer "F.Cu") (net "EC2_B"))
 (segment (start 211.459895 33.022) (end 211.279894 33.022) (width 0.2) (layer "F.Cu") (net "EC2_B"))
 (segment (start 212.082 29.869786) (end 212.082 32.399895) (width 0.2) (layer "F.Cu") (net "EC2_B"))
 (segment (start 177.301894 67) (end 165.75 67) (width 0.2) (layer "F.Cu") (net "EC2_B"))
 (segment (start 210.218786 29.609) (end 211.821214 29.609) (width 0.2) (layer "F.Cu") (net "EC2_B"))
 (segment (start 212.082 32.399895) (end 211.459895 33.022) (width 0.2) (layer "F.Cu") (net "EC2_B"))
 (segment (start 205.05 32.85) (end 205.94 31.96) (width 0.2) (layer "F.Cu") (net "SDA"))
 (segment (start 159.8 63.04) (end 188.89 33.95) (width 0.2) (layer "F.Cu") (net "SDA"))
 (segment (start 188.89 33.95) (end 205.05 33.95) (width 0.2) (layer "F.Cu") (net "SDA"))
 (segment (start 205.05 33.95) (end 205.05 32.85) (width 0.2) (layer "F.Cu") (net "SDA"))
 (segment (start 205.94 31.96) (end 205.94 33.69) (width 0.2) (layer "B.Cu") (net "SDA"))
 (segment (start 215.67 62.97) (end 217.2 62.97) (width 0.2) (layer "B.Cu") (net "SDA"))
 (segment (start 214.55 65.62) (end 214.55 126.01) (width 0.2) (layer "B.Cu") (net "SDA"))
 (segment (start 205.94 33.69) (end 217.75 45.5) (width 0.2) (layer "B.Cu") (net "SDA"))
 (segment (start 215.25 57.54) (end 215.25 62.55) (width 0.2) (layer "B.Cu") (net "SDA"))
 (segment (start 163.5 63.7) (end 162.84 63.04) (width 0.2) (layer "B.Cu") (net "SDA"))
 (segment (start 217.75 45.5) (end 217.75 55.04) (width 0.2) (layer "B.Cu") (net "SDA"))
 (segment (start 162.84 63.04) (end 159.8 63.04) (width 0.2) (layer "B.Cu") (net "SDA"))
 (segment (start 217.2 62.97) (end 214.55 65.62) (width 0.2) (layer "B.Cu") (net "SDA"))
 (segment (start 163.5 124.76) (end 163.5 63.7) (width 0.2) (layer "B.Cu") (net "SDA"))
 (segment (start 214.55 126.01) (end 217 128.46) (width 0.2) (layer "B.Cu") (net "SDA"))
 (segment (start 215.25 62.55) (end 215.67 62.97) (width 0.2) (layer "B.Cu") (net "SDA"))
 (segment (start 217.75 55.04) (end 215.25 57.54) (width 0.2) (layer "B.Cu") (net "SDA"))
 (segment (start 159.8 128.46) (end 163.5 124.76) (width 0.2) (layer "B.Cu") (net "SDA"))
 (segment (start 218.15 129.85) (end 218.15 66.46) (width 0.2) (layer "B.Cu") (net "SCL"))
 (segment (start 204.462 30.898) (end 203.4 31.96) (width 0.2) (layer "B.Cu") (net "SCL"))
 (segment (start 203.4 31.96) (end 202.338 33.022) (width 0.2) (layer "B.Cu") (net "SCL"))
 (segment (start 159.8 65.58) (end 158.65 64.43) (width 0.2) (layer "B.Cu") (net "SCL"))
 (segment (start 217 131) (end 218.15 129.85) (width 0.2) (layer "B.Cu") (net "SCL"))
 (segment (start 158.65 60.023654) (end 158.65 62.563654) (width 0.2) (layer "B.Cu") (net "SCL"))
 (segment (start 160.8 59.35) (end 159.323654 59.35) (width 0.2) (layer "B.Cu") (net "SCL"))
 (segment (start 164.15 127.65) (end 160.8 131) (width 0.2) (layer "B.Cu") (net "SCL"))
 (segment (start 160.8 131) (end 159.8 131) (width 0.2) (layer "B.Cu") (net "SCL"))
 (segment (start 218.35 44.05) (end 207.05 32.75) (width 0.2) (layer "B.Cu") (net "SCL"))
 (segment (start 202.338 33.022) (end 187.128 33.022) (width 0.2) (layer "B.Cu") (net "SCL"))
 (segment (start 218.15 66.46) (end 217.2 65.51) (width 0.2) (layer "B.Cu") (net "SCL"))
 (segment (start 187.128 33.022) (end 160.8 59.35) (width 0.2) (layer "B.Cu") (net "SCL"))
 (segment (start 158.65 64.43) (end 158.65 62.563654) (width 0.2) (layer "B.Cu") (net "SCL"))
 (segment (start 162.255686 61.89) (end 164.15 63.784314) (width 0.2) (layer "B.Cu") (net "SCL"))
 (segment (start 159.323654 61.89) (end 162.255686 61.89) (width 0.2) (layer "B.Cu") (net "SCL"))
 (segment (start 158.65 62.563654) (end 159.323654 61.89) (width 0.2) (layer "B.Cu") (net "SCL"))
 (segment (start 207.05 32.75) (end 207.05 31.568105) (width 0.2) (layer "B.Cu") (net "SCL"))
 (segment (start 217.2 65.51) (end 218.35 64.36) (width 0.2) (layer "B.Cu") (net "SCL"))
 (segment (start 218.35 64.36) (end 218.35 44.05) (width 0.2) (layer "B.Cu") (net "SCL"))
 (segment (start 206.379895 30.898) (end 204.462 30.898) (width 0.2) (layer "B.Cu") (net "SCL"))
 (segment (start 164.15 63.784314) (end 164.15 127.65) (width 0.2) (layer "B.Cu") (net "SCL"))
 (segment (start 207.05 31.568105) (end 206.379895 30.898) (width 0.2) (layer "B.Cu") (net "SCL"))
 (segment (start 159.323654 59.35) (end 158.65 60.023654) (width 0.2) (layer "B.Cu") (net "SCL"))
 (segment (start 203.25 33.35) (end 203.2 33.3) (width 0.2) (layer "F.Cu") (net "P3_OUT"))
 (segment (start 202.2 33.3) (end 200.86 31.96) (width 0.2) (layer "F.Cu") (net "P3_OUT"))
 (segment (start 203.2 33.3) (end 202.2 33.3) (width 0.2) (layer "F.Cu") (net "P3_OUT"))
 (via (at 203.25 33.35) (size 0.6) (drill 0.3) (layers "F.Cu" "B.Cu") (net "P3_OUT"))
 (segment (start 202.7 33.9) (end 203.25 33.35) (width 0.2) (layer "B.Cu") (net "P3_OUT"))
 (segment (start 211.2 44.45) (end 202.7 35.95) (width 0.2) (layer "B.Cu") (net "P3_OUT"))
 (segment (start 212.082 46.760105) (end 211.459895 46.138) (width 0.2) (layer "B.Cu") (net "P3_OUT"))
 (segment (start 211.459895 46.138) (end 211.2 46.138) (width 0.2) (layer "B.Cu") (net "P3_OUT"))
 (segment (start 211.2 48.262) (end 211.459895 48.262) (width 0.2) (layer "B.Cu") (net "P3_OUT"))
 (segment (start 212.082 47.639895) (end 212.082 46.760105) (width 0.2) (layer "B.Cu") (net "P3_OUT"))
 (segment (start 211.2 48.732209) (end 211.2 48.262) (width 0.2) (layer "B.Cu") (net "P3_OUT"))
 (segment (start 191.15 80.3) (end 205.7 80.3) (width 0.2) (layer "B.Cu") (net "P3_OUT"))
 (segment (start 211.2 74.8) (end 211.2 72.965686) (width 0.2) (layer "B.Cu") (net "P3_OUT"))
 (segment (start 202.7 35.95) (end 202.7 33.9) (width 0.2) (layer "B.Cu") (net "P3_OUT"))
 (segment (start 211.459895 48.262) (end 212.082 47.639895) (width 0.2) (layer "B.Cu") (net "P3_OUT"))
 (segment (start 211.2 72.965686) (end 211.45 72.715685) (width 0.2) (layer "B.Cu") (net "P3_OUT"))
 (segment (start 205.7 80.3) (end 211.2 74.8) (width 0.2) (layer "B.Cu") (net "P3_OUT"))
 (segment (start 211.45 72.715685) (end 211.45 48.982209) (width 0.2) (layer "B.Cu") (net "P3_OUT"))
 (segment (start 189.95 79.1) (end 191.15 80.3) (width 0.2) (layer "B.Cu") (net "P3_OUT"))
 (segment (start 211.2 46.138) (end 211.2 44.45) (width 0.2) (layer "B.Cu") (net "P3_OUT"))
 (segment (start 211.45 48.982209) (end 211.2 48.732209) (width 0.2) (layer "B.Cu") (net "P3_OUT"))
 (segment (start 209.542 46.760105) (end 208.919895 46.138) (width 0.2) (layer "B.Cu") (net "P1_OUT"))
 (segment (start 204.462 46.138) (end 203.4 47.2) (width 0.2) (layer "B.Cu") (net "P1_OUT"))
 (segment (start 211.05 72.55) (end 211.05 49.147895) (width 0.2) (layer "B.Cu") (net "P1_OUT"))
 (segment (start 209.542 47.639895) (end 209.542 46.760105) (width 0.2) (layer "B.Cu") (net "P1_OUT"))
 (segment (start 211.05 49.147895) (end 209.542 47.639895) (width 0.2) (layer "B.Cu") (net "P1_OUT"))
 (segment (start 204.5 79.1) (end 211.05 72.55) (width 0.2) (layer "B.Cu") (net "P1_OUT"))
 (segment (start 208.919895 46.138) (end 204.462 46.138) (width 0.2) (layer "B.Cu") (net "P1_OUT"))
 (segment (start 208 49.15) (end 208.48 48.67) (width 0.2) (layer "B.Cu") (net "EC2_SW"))
 (segment (start 187.641895 67) (end 205.491895 49.15) (width 0.2) (layer "B.Cu") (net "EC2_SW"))
 (segment (start 208.48 48.67) (end 208.48 47.2) (width 0.2) (layer "B.Cu") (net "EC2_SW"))
 (segment (start 180.25 67) (end 187.641895 67) (width 0.2) (layer "B.Cu") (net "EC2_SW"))
 (segment (start 205.491895 49.15) (end 208 49.15) (width 0.2) (layer "B.Cu") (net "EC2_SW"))
 (segment (start 160.81 57.96) (end 159.8 57.96) (width 0.2) (layer "F.Cu") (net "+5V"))
 (segment (start 159.8 123.38) (end 160.55 122.63) (width 0.2) (layer "F.Cu") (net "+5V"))
 (segment (start 159.8 58.65) (end 159.8 57.96) (width 0.2) (layer "F.Cu") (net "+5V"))
 (segment (start 213.9 120.28) (end 217 123.38) (width 0.2) (layer "F.Cu") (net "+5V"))
 (segment (start 216.1 48.035) (end 216.1 56.79) (width 0.2) (layer "F.Cu") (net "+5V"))
 (segment (start 188.95 35) (end 205 35) (width 0.2) (layer "F.Cu") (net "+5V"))
 (segment (start 217.2 57.89) (end 213.9 61.19) (width 0.2) (layer "F.Cu") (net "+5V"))
 (segment (start 161.924265 59.074265) (end 160.81 57.96) (width 0.2) (layer "F.Cu") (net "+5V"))
 (segment (start 213.9 61.19) (end 213.9 120.28) (width 0.2) (layer "F.Cu") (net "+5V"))
 (segment (start 160.55 69.25) (end 163.55 66.25) (width 0.2) (layer "F.Cu") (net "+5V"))
 (segment (start 163.55 66.25) (end 163.55 60.4) (width 0.2) (layer "F.Cu") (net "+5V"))
 (segment (start 160.55 122.63) (end 160.55 69.25) (width 0.2) (layer "F.Cu") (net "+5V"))
 (segment (start 163.55 60.4) (end 188.95 35) (width 0.2) (layer "F.Cu") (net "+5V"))
 (segment (start 216.1 56.79) (end 217.2 57.89) (width 0.2) (layer "F.Cu") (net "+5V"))
 (segment (start 160.55 69.25) (end 160.55 69) (width 0.2) (layer "F.Cu") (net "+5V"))
 (via (at 161.924265 59.074265) (size 0.6) (drill 0.3) (layers "F.Cu" "B.Cu") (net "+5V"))
 (via (at 205 35) (size 0.6) (drill 0.3) (layers "F.Cu" "B.Cu") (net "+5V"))
 (via (at 163.55 60.4) (size 0.6) (drill 0.3) (layers "F.Cu" "B.Cu") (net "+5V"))
 (segment (start 163.55 60.4) (end 163.25 60.4) (width 0.2) (layer "B.Cu") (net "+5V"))
 (segment (start 205 36.1) (end 216.1 47.2) (width 0.2) (layer "B.Cu") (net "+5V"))
 (segment (start 163.25 60.4) (end 161.924265 59.074265) (width 0.2) (layer "B.Cu") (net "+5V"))
 (segment (start 205 35) (end 205 36.1) (width 0.2) (layer "B.Cu") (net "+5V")))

